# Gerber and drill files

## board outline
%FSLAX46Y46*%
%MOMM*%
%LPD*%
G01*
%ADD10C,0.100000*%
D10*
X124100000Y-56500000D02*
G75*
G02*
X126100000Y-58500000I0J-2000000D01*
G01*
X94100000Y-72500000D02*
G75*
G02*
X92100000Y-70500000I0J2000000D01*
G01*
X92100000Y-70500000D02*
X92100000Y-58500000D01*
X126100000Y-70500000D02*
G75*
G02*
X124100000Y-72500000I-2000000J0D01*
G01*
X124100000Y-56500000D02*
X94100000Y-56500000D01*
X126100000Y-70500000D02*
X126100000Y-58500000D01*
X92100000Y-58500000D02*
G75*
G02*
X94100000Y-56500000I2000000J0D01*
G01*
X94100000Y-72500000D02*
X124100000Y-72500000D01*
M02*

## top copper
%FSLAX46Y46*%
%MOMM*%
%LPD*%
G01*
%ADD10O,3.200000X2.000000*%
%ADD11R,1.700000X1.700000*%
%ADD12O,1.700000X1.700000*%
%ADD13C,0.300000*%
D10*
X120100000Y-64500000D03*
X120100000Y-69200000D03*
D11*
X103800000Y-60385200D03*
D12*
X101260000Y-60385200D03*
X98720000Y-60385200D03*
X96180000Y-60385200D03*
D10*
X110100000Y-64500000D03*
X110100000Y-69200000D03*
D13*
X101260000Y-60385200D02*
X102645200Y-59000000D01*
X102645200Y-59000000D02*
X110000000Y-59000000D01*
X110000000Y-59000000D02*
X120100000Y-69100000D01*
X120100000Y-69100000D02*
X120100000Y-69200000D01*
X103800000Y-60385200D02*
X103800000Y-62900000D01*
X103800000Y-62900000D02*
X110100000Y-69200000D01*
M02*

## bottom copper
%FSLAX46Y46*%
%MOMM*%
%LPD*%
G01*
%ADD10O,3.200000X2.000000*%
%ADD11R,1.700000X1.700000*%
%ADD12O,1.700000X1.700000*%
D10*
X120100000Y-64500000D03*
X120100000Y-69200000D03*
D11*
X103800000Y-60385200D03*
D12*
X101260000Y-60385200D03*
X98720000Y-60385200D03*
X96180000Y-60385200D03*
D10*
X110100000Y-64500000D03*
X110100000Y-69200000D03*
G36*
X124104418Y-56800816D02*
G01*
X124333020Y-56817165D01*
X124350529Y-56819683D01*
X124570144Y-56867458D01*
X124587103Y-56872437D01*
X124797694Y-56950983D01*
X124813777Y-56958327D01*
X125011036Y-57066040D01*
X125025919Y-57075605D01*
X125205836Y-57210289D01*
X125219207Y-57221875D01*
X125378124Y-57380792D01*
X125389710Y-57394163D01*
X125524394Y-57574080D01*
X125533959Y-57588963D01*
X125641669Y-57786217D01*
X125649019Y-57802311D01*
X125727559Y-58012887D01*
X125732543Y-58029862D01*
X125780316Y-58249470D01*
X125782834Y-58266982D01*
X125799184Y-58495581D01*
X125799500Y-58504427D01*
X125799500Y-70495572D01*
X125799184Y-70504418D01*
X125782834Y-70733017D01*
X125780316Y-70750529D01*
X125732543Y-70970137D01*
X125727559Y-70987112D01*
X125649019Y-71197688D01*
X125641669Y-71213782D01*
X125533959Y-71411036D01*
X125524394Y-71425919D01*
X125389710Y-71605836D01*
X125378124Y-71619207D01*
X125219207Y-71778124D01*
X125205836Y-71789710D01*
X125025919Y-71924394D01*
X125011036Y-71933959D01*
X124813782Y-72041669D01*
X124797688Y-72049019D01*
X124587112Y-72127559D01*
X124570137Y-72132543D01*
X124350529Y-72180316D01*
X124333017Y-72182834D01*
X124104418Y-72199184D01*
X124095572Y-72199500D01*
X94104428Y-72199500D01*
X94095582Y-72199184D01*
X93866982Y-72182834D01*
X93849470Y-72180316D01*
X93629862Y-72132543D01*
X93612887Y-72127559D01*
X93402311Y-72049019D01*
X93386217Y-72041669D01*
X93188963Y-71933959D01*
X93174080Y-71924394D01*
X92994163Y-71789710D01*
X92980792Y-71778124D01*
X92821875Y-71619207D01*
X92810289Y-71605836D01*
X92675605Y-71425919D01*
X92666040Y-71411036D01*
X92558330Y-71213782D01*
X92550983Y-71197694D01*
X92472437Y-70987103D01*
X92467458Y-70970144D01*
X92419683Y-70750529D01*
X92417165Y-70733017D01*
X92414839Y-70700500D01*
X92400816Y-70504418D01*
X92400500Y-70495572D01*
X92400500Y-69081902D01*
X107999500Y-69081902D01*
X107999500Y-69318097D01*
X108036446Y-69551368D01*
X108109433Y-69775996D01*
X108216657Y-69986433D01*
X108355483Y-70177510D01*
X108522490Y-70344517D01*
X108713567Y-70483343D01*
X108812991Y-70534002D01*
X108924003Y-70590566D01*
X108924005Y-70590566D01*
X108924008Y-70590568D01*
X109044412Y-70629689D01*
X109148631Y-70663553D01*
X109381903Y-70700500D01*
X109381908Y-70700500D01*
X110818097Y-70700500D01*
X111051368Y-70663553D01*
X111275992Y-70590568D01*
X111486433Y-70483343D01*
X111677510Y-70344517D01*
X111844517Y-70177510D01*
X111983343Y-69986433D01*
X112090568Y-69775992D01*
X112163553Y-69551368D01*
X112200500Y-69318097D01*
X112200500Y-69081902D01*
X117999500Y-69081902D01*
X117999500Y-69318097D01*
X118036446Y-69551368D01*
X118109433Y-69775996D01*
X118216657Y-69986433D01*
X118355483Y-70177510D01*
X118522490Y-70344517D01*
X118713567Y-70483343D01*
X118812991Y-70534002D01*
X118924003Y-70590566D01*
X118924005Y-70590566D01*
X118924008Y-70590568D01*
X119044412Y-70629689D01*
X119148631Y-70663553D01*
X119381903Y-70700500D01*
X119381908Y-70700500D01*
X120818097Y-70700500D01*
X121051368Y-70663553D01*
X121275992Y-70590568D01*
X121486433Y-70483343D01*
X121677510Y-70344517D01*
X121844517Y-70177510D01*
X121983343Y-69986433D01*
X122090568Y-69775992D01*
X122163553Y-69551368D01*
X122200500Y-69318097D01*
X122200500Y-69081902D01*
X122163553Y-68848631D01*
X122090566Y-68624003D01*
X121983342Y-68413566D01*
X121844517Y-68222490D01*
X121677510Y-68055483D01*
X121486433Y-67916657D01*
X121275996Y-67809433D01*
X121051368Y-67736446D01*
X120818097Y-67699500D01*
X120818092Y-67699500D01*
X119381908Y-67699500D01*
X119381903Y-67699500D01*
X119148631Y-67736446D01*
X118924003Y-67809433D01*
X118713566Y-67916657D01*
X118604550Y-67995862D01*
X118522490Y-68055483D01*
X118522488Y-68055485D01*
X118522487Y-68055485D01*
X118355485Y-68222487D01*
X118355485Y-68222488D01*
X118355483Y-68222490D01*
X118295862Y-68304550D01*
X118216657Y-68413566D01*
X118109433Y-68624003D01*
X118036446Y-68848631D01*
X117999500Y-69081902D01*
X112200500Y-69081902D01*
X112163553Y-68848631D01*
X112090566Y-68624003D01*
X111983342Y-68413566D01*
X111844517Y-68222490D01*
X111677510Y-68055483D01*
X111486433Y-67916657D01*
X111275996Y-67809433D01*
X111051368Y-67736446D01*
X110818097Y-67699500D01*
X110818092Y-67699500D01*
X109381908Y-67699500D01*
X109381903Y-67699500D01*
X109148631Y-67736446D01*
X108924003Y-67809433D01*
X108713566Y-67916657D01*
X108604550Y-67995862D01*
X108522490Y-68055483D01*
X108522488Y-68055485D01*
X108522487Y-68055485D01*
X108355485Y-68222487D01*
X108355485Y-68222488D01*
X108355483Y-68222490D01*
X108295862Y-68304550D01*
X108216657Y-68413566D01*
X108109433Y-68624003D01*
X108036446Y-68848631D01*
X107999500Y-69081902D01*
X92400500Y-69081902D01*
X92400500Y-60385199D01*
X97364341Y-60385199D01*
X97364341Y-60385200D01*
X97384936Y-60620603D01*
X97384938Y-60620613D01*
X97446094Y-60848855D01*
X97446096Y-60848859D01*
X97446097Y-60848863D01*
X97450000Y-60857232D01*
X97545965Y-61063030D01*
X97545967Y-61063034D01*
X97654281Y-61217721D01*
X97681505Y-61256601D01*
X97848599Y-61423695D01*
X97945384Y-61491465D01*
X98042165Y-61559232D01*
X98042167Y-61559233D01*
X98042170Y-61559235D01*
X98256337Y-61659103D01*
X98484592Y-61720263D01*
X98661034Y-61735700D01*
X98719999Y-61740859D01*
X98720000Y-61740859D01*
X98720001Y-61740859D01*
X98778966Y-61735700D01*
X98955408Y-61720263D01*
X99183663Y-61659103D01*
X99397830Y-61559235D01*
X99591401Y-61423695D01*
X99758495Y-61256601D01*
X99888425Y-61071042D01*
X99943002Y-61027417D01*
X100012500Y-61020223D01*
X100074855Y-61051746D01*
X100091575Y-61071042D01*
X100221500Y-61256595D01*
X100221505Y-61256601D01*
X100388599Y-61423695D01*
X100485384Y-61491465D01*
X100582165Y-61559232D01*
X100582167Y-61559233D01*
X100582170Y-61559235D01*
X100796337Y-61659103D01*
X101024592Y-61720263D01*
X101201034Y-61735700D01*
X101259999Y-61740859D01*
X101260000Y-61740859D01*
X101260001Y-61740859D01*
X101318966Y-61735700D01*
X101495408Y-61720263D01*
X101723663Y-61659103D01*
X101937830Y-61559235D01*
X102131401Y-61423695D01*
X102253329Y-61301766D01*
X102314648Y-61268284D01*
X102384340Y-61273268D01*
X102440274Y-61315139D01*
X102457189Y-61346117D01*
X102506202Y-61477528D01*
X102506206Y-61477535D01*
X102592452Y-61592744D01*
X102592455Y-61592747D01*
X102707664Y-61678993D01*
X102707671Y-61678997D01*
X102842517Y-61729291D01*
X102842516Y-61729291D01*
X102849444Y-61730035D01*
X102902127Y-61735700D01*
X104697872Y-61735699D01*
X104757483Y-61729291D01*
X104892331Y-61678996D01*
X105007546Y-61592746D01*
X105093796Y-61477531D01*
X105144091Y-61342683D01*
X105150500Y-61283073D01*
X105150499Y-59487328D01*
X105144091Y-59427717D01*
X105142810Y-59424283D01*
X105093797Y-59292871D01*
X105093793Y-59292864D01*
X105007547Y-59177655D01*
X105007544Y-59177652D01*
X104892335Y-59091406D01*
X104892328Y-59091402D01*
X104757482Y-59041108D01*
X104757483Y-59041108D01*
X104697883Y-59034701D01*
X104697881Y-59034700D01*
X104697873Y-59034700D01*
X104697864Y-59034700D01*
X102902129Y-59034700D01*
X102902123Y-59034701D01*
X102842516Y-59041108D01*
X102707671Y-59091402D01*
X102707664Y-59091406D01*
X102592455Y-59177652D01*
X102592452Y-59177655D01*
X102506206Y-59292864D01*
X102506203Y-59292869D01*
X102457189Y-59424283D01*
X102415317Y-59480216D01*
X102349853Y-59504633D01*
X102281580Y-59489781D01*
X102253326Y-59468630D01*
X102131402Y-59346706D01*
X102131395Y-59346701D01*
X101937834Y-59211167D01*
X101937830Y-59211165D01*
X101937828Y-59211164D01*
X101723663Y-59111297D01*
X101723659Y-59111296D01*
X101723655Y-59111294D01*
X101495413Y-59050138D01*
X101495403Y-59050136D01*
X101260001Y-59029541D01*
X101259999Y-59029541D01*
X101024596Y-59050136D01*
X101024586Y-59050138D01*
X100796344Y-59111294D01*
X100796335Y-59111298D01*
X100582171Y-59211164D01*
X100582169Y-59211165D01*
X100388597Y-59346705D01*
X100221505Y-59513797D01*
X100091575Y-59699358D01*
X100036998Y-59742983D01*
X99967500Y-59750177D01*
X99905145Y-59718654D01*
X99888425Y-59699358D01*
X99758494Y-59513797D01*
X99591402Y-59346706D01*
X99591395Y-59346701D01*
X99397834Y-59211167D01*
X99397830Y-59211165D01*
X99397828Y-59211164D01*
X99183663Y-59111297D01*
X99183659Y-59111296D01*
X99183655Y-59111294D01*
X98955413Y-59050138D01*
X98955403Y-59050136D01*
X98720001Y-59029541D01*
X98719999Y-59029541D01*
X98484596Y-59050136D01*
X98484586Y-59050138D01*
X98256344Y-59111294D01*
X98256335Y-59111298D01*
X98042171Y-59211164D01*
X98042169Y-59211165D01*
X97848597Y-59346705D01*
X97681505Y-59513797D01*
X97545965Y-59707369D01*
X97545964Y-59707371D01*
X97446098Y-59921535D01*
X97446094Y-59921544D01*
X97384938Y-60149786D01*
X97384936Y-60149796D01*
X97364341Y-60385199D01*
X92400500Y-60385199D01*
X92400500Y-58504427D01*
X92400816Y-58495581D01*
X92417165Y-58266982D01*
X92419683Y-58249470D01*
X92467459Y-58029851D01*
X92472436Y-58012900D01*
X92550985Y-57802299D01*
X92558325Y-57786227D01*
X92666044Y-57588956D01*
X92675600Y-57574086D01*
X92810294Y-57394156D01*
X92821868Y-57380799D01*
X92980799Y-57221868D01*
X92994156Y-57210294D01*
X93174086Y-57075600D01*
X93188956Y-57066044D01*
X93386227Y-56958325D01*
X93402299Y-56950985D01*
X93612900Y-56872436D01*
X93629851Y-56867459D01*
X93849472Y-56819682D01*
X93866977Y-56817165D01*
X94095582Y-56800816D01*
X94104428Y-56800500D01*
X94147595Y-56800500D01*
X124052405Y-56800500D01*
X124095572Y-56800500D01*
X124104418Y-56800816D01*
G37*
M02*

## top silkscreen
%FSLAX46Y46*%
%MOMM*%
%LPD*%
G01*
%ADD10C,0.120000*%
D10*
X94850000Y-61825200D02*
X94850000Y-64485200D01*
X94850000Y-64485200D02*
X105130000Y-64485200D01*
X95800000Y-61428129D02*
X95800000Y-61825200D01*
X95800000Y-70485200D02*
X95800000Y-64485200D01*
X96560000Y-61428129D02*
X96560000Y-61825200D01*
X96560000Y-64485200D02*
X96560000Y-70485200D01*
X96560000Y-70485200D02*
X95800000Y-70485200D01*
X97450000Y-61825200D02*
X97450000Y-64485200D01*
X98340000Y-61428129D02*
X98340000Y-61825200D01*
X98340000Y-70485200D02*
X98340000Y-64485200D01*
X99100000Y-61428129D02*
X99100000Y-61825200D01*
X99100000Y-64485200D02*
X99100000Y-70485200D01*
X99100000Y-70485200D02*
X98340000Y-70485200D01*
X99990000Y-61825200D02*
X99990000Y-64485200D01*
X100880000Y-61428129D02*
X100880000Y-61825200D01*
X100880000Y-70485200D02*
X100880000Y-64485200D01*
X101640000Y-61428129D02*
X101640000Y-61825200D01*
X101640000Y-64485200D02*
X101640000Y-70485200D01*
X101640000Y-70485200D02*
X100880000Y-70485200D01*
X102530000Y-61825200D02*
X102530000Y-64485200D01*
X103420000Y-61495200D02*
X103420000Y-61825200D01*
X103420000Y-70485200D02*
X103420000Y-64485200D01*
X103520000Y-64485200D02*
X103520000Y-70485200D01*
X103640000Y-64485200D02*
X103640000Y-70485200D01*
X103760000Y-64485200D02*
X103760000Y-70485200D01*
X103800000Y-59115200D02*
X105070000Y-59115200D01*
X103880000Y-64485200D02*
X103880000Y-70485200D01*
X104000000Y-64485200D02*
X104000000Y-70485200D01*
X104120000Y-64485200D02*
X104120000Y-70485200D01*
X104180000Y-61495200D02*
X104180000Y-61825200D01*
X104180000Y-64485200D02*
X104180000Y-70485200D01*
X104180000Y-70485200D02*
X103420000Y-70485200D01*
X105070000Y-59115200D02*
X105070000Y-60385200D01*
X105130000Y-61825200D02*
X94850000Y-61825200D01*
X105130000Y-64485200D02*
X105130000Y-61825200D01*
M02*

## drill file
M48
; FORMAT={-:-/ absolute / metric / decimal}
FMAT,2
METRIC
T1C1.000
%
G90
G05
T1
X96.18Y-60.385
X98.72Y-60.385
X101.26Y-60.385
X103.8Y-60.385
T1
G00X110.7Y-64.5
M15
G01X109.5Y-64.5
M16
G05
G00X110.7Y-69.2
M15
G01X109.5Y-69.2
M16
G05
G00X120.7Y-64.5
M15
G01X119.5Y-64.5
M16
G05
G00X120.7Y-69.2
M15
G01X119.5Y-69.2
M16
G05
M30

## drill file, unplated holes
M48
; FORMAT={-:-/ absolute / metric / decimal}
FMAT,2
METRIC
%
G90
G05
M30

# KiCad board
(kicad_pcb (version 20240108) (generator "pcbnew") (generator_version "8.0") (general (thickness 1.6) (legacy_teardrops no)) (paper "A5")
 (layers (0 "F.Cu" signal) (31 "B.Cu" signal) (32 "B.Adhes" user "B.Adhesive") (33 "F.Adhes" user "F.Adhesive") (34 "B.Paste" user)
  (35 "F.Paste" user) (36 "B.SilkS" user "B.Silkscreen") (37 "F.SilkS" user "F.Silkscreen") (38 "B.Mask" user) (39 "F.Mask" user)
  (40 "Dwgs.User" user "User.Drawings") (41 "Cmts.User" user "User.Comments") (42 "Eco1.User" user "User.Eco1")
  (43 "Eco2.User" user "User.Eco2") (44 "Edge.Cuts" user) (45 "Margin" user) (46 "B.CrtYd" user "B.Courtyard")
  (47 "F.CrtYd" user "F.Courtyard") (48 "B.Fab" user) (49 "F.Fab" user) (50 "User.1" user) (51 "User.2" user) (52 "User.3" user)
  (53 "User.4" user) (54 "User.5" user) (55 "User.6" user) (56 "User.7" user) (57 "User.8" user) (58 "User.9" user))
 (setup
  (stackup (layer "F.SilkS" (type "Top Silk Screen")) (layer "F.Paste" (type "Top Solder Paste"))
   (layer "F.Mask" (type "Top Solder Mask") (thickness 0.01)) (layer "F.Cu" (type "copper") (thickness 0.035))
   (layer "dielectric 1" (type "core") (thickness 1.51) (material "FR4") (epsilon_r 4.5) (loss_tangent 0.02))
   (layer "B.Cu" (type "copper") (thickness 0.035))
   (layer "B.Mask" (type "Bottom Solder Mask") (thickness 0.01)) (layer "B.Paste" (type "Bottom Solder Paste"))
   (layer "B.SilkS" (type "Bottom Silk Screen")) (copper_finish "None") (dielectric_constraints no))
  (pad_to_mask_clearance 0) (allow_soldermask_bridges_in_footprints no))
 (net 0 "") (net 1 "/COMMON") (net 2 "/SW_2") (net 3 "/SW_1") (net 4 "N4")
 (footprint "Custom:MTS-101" (layer "F.Cu") (at 120.1 64.5 180)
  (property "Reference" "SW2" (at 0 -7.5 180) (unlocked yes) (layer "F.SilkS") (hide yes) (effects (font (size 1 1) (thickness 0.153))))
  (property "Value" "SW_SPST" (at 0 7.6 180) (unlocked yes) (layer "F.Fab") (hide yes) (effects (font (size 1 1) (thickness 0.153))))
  (pad "1" thru_hole oval (at 0 0 180) (size 3.2 2) (drill oval 2.2 1) (layers "*.Cu" "*.Mask") (remove_unused_layers no) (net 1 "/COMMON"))
  (pad "2" thru_hole oval (at 0 -4.7 180) (size 3.2 2) (drill oval 2.2 1) (layers "*.Cu" "*.Mask") (remove_unused_layers no) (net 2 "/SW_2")))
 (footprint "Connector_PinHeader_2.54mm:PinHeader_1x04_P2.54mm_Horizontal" (layer "F.Cu") (at 103.8 60.3852 -90)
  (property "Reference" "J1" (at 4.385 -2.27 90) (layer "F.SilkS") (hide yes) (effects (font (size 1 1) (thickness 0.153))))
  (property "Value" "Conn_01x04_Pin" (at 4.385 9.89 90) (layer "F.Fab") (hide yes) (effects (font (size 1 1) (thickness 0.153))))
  (fp_line (start 1.44 8.95) (end 4.1 8.95) (stroke (width 0.12) (type solid)) (layer "F.SilkS"))
  (fp_line (start 4.1 8.95) (end 4.1 -1.33) (stroke (width 0.12) (type solid)) (layer "F.SilkS"))
  (fp_line (start 1.042929 8) (end 1.44 8) (stroke (width 0.12) (type solid)) (layer "F.SilkS"))
  (fp_line (start 10.1 8) (end 4.1 8) (stroke (width 0.12) (type solid)) (layer "F.SilkS"))
  (fp_line (start 1.042929 7.24) (end 1.44 7.24) (stroke (width 0.12) (type solid)) (layer "F.SilkS"))
  (fp_line (start 4.1 7.24) (end 10.1 7.24) (stroke (width 0.12) (type solid)) (layer "F.SilkS"))
  (fp_line (start 10.1 7.24) (end 10.1 8) (stroke (width 0.12) (type solid)) (layer "F.SilkS"))
  (fp_line (start 1.44 6.35) (end 4.1 6.35) (stroke (width 0.12) (type solid)) (layer "F.SilkS"))
  (fp_line (start 1.042929 5.46) (end 1.44 5.46) (stroke (width 0.12) (type solid)) (layer "F.SilkS"))
  (fp_line (start 10.1 5.46) (end 4.1 5.46) (stroke (width 0.12) (type solid)) (layer "F.SilkS"))
  (fp_line (start 1.042929 4.7) (end 1.44 4.7) (stroke (width 0.12) (type solid)) (layer "F.SilkS"))
  (fp_line (start 4.1 4.7) (end 10.1 4.7) (stroke (width 0.12) (type solid)) (layer "F.SilkS"))
  (fp_line (start 10.1 4.7) (end 10.1 5.46) (stroke (width 0.12) (type solid)) (layer "F.SilkS"))
  (fp_line (start 1.44 3.81) (end 4.1 3.81) (stroke (width 0.12) (type solid)) (layer "F.SilkS"))
  (fp_line (start 1.042929 2.92) (end 1.44 2.92) (stroke (width 0.12) (type solid)) (layer "F.SilkS"))
  (fp_line (start 10.1 2.92) (end 4.1 2.92) (stroke (width 0.12) (type solid)) (layer "F.SilkS"))
  (fp_line (start 1.042929 2.16) (end 1.44 2.16) (stroke (width 0.12) (type solid)) (layer "F.SilkS"))
  (fp_line (start 4.1 2.16) (end 10.1 2.16) (stroke (width 0.12) (type solid)) (layer "F.SilkS"))
  (fp_line (start 10.1 2.16) (end 10.1 2.92) (stroke (width 0.12) (type solid)) (layer "F.SilkS"))
  (fp_line (start 1.44 1.27) (end 4.1 1.27) (stroke (width 0.12) (type solid)) (layer "F.SilkS"))
  (fp_line (start 1.11 0.38) (end 1.44 0.38) (stroke (width 0.12) (type solid)) (layer "F.SilkS"))
  (fp_line (start 10.1 0.38) (end 4.1 0.38) (stroke (width 0.12) (type solid)) (layer "F.SilkS"))
  (fp_line (start 4.1 0.28) (end 10.1 0.28) (stroke (width 0.12) (type solid)) (layer "F.SilkS"))
  (fp_line (start 4.1 0.16) (end 10.1 0.16) (stroke (width 0.12) (type solid)) (layer "F.SilkS"))
  (fp_line (start 4.1 0.04) (end 10.1 0.04) (stroke (width 0.12) (type solid)) (layer "F.SilkS"))
  (fp_line (start -1.27 0) (end -1.27 -1.27) (stroke (width 0.12) (type solid)) (layer "F.SilkS"))
  (fp_line (start 4.1 -0.08) (end 10.1 -0.08) (stroke (width 0.12) (type solid)) (layer "F.SilkS"))
  (fp_line (start 4.1 -0.2) (end 10.1 -0.2) (stroke (width 0.12) (type solid)) (layer "F.SilkS"))
  (fp_line (start 4.1 -0.32) (end 10.1 -0.32) (stroke (width 0.12) (type solid)) (layer "F.SilkS"))
  (fp_line (start 1.11 -0.38) (end 1.44 -0.38) (stroke (width 0.12) (type solid)) (layer "F.SilkS"))
  (fp_line (start 4.1 -0.38) (end 10.1 -0.38) (stroke (width 0.12) (type solid)) (layer "F.SilkS"))
  (fp_line (start 10.1 -0.38) (end 10.1 0.38) (stroke (width 0.12) (type solid)) (layer "F.SilkS"))
  (fp_line (start -1.27 -1.27) (end 0 -1.27) (stroke (width 0.12) (type solid)) (layer "F.SilkS"))
  (fp_line (start 1.44 -1.33) (end 1.44 8.95) (stroke (width 0.12) (type solid)) (layer "F.SilkS"))
  (fp_line (start 4.1 -1.33) (end 1.44 -1.33) (stroke (width 0.12) (type solid)) (layer "F.SilkS"))
  (pad "1" thru_hole rect (at 0 0 270) (size 1.7 1.7) (drill 1) (layers "*.Cu" "*.Mask") (remove_unused_layers no) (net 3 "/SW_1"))
  (pad "2" thru_hole oval (at 0 2.54 270) (size 1.7 1.7) (drill 1) (layers "*.Cu" "*.Mask") (remove_unused_layers no) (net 2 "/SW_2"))
  (pad "3" thru_hole oval (at 0 5.08 270) (size 1.7 1.7) (drill 1) (layers "*.Cu" "*.Mask") (remove_unused_layers no) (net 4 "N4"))
  (pad "4" thru_hole oval (at 0 7.62 270) (size 1.7 1.7) (drill 1) (layers "*.Cu" "*.Mask") (remove_unused_layers no) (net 1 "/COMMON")))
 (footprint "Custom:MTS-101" (layer "F.Cu") (at 110.1 64.5 180)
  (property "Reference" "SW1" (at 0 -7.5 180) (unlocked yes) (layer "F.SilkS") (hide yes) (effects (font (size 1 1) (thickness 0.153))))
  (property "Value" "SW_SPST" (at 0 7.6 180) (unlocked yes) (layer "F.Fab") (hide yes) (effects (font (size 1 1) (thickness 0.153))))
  (pad "1" thru_hole oval (at 0 0 180) (size 3.2 2) (drill oval 2.2 1) (layers "*.Cu" "*.Mask") (remove_unused_layers no) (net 1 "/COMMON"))
  (pad "2" thru_hole oval (at 0 -4.7 180) (size 3.2 2) (drill oval 2.2 1) (layers "*.Cu" "*.Mask") (remove_unused_layers no) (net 3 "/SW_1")))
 (gr_arc (start 124.1 56.5) (mid 125.514214 57.085786) (end 126.1 58.5) (stroke (width 0.1) (type default)) (layer "Edge.Cuts"))
 (gr_arc (start 94.1 72.5) (mid 92.685786 71.914214) (end 92.1 70.5) (stroke (width 0.1) (type default)) (layer "Edge.Cuts"))
 (gr_line (start 92.1 70.5) (end 92.1 58.5) (stroke (width 0.1) (type default)) (layer "Edge.Cuts"))
 (gr_arc (start 126.1 70.5) (mid 125.514214 71.914214) (end 124.1 72.5) (stroke (width 0.1) (type default)) (layer "Edge.Cuts"))
 (gr_line (start 124.1 56.5) (end 94.1 56.5) (stroke (width 0.1) (type default)) (layer "Edge.Cuts"))
 (gr_line (start 126.1 70.5) (end 126.1 58.5) (stroke (width 0.1) (type default)) (layer "Edge.Cuts"))
 (gr_arc (start 92.1 58.5) (mid 92.685786 57.085786) (end 94.1 56.5) (stroke (width 0.1) (type default)) (layer "Edge.Cuts"))
 (gr_line (start 94.1 72.5) (end 124.1 72.5) (stroke (width 0.1) (type default)) (layer "Edge.Cuts"))
 (segment (start 103.8 60.3852) (end 103.8 62.9) (width 0.3) (layer "F.Cu") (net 3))
 (segment (start 103.8 62.9) (end 110.1 69.2) (width 0.3) (layer "F.Cu") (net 3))
 (segment (start 110 59) (end 120.1 69.1) (width 0.3) (layer "F.Cu") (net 2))
 (segment (start 102.6452 59) (end 110 59) (width 0.3) (layer "F.Cu") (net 2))
 (segment (start 120.1 69.1) (end 120.1 69.2) (width 0.3) (layer "F.Cu") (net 2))
 (segment (start 101.26 60.3852) (end 102.6452 59) (width 0.3) (layer "F.Cu") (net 2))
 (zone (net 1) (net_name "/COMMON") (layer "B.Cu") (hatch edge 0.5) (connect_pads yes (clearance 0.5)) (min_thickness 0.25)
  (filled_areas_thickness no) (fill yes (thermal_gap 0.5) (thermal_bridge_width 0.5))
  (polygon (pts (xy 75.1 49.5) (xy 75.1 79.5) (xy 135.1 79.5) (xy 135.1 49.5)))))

